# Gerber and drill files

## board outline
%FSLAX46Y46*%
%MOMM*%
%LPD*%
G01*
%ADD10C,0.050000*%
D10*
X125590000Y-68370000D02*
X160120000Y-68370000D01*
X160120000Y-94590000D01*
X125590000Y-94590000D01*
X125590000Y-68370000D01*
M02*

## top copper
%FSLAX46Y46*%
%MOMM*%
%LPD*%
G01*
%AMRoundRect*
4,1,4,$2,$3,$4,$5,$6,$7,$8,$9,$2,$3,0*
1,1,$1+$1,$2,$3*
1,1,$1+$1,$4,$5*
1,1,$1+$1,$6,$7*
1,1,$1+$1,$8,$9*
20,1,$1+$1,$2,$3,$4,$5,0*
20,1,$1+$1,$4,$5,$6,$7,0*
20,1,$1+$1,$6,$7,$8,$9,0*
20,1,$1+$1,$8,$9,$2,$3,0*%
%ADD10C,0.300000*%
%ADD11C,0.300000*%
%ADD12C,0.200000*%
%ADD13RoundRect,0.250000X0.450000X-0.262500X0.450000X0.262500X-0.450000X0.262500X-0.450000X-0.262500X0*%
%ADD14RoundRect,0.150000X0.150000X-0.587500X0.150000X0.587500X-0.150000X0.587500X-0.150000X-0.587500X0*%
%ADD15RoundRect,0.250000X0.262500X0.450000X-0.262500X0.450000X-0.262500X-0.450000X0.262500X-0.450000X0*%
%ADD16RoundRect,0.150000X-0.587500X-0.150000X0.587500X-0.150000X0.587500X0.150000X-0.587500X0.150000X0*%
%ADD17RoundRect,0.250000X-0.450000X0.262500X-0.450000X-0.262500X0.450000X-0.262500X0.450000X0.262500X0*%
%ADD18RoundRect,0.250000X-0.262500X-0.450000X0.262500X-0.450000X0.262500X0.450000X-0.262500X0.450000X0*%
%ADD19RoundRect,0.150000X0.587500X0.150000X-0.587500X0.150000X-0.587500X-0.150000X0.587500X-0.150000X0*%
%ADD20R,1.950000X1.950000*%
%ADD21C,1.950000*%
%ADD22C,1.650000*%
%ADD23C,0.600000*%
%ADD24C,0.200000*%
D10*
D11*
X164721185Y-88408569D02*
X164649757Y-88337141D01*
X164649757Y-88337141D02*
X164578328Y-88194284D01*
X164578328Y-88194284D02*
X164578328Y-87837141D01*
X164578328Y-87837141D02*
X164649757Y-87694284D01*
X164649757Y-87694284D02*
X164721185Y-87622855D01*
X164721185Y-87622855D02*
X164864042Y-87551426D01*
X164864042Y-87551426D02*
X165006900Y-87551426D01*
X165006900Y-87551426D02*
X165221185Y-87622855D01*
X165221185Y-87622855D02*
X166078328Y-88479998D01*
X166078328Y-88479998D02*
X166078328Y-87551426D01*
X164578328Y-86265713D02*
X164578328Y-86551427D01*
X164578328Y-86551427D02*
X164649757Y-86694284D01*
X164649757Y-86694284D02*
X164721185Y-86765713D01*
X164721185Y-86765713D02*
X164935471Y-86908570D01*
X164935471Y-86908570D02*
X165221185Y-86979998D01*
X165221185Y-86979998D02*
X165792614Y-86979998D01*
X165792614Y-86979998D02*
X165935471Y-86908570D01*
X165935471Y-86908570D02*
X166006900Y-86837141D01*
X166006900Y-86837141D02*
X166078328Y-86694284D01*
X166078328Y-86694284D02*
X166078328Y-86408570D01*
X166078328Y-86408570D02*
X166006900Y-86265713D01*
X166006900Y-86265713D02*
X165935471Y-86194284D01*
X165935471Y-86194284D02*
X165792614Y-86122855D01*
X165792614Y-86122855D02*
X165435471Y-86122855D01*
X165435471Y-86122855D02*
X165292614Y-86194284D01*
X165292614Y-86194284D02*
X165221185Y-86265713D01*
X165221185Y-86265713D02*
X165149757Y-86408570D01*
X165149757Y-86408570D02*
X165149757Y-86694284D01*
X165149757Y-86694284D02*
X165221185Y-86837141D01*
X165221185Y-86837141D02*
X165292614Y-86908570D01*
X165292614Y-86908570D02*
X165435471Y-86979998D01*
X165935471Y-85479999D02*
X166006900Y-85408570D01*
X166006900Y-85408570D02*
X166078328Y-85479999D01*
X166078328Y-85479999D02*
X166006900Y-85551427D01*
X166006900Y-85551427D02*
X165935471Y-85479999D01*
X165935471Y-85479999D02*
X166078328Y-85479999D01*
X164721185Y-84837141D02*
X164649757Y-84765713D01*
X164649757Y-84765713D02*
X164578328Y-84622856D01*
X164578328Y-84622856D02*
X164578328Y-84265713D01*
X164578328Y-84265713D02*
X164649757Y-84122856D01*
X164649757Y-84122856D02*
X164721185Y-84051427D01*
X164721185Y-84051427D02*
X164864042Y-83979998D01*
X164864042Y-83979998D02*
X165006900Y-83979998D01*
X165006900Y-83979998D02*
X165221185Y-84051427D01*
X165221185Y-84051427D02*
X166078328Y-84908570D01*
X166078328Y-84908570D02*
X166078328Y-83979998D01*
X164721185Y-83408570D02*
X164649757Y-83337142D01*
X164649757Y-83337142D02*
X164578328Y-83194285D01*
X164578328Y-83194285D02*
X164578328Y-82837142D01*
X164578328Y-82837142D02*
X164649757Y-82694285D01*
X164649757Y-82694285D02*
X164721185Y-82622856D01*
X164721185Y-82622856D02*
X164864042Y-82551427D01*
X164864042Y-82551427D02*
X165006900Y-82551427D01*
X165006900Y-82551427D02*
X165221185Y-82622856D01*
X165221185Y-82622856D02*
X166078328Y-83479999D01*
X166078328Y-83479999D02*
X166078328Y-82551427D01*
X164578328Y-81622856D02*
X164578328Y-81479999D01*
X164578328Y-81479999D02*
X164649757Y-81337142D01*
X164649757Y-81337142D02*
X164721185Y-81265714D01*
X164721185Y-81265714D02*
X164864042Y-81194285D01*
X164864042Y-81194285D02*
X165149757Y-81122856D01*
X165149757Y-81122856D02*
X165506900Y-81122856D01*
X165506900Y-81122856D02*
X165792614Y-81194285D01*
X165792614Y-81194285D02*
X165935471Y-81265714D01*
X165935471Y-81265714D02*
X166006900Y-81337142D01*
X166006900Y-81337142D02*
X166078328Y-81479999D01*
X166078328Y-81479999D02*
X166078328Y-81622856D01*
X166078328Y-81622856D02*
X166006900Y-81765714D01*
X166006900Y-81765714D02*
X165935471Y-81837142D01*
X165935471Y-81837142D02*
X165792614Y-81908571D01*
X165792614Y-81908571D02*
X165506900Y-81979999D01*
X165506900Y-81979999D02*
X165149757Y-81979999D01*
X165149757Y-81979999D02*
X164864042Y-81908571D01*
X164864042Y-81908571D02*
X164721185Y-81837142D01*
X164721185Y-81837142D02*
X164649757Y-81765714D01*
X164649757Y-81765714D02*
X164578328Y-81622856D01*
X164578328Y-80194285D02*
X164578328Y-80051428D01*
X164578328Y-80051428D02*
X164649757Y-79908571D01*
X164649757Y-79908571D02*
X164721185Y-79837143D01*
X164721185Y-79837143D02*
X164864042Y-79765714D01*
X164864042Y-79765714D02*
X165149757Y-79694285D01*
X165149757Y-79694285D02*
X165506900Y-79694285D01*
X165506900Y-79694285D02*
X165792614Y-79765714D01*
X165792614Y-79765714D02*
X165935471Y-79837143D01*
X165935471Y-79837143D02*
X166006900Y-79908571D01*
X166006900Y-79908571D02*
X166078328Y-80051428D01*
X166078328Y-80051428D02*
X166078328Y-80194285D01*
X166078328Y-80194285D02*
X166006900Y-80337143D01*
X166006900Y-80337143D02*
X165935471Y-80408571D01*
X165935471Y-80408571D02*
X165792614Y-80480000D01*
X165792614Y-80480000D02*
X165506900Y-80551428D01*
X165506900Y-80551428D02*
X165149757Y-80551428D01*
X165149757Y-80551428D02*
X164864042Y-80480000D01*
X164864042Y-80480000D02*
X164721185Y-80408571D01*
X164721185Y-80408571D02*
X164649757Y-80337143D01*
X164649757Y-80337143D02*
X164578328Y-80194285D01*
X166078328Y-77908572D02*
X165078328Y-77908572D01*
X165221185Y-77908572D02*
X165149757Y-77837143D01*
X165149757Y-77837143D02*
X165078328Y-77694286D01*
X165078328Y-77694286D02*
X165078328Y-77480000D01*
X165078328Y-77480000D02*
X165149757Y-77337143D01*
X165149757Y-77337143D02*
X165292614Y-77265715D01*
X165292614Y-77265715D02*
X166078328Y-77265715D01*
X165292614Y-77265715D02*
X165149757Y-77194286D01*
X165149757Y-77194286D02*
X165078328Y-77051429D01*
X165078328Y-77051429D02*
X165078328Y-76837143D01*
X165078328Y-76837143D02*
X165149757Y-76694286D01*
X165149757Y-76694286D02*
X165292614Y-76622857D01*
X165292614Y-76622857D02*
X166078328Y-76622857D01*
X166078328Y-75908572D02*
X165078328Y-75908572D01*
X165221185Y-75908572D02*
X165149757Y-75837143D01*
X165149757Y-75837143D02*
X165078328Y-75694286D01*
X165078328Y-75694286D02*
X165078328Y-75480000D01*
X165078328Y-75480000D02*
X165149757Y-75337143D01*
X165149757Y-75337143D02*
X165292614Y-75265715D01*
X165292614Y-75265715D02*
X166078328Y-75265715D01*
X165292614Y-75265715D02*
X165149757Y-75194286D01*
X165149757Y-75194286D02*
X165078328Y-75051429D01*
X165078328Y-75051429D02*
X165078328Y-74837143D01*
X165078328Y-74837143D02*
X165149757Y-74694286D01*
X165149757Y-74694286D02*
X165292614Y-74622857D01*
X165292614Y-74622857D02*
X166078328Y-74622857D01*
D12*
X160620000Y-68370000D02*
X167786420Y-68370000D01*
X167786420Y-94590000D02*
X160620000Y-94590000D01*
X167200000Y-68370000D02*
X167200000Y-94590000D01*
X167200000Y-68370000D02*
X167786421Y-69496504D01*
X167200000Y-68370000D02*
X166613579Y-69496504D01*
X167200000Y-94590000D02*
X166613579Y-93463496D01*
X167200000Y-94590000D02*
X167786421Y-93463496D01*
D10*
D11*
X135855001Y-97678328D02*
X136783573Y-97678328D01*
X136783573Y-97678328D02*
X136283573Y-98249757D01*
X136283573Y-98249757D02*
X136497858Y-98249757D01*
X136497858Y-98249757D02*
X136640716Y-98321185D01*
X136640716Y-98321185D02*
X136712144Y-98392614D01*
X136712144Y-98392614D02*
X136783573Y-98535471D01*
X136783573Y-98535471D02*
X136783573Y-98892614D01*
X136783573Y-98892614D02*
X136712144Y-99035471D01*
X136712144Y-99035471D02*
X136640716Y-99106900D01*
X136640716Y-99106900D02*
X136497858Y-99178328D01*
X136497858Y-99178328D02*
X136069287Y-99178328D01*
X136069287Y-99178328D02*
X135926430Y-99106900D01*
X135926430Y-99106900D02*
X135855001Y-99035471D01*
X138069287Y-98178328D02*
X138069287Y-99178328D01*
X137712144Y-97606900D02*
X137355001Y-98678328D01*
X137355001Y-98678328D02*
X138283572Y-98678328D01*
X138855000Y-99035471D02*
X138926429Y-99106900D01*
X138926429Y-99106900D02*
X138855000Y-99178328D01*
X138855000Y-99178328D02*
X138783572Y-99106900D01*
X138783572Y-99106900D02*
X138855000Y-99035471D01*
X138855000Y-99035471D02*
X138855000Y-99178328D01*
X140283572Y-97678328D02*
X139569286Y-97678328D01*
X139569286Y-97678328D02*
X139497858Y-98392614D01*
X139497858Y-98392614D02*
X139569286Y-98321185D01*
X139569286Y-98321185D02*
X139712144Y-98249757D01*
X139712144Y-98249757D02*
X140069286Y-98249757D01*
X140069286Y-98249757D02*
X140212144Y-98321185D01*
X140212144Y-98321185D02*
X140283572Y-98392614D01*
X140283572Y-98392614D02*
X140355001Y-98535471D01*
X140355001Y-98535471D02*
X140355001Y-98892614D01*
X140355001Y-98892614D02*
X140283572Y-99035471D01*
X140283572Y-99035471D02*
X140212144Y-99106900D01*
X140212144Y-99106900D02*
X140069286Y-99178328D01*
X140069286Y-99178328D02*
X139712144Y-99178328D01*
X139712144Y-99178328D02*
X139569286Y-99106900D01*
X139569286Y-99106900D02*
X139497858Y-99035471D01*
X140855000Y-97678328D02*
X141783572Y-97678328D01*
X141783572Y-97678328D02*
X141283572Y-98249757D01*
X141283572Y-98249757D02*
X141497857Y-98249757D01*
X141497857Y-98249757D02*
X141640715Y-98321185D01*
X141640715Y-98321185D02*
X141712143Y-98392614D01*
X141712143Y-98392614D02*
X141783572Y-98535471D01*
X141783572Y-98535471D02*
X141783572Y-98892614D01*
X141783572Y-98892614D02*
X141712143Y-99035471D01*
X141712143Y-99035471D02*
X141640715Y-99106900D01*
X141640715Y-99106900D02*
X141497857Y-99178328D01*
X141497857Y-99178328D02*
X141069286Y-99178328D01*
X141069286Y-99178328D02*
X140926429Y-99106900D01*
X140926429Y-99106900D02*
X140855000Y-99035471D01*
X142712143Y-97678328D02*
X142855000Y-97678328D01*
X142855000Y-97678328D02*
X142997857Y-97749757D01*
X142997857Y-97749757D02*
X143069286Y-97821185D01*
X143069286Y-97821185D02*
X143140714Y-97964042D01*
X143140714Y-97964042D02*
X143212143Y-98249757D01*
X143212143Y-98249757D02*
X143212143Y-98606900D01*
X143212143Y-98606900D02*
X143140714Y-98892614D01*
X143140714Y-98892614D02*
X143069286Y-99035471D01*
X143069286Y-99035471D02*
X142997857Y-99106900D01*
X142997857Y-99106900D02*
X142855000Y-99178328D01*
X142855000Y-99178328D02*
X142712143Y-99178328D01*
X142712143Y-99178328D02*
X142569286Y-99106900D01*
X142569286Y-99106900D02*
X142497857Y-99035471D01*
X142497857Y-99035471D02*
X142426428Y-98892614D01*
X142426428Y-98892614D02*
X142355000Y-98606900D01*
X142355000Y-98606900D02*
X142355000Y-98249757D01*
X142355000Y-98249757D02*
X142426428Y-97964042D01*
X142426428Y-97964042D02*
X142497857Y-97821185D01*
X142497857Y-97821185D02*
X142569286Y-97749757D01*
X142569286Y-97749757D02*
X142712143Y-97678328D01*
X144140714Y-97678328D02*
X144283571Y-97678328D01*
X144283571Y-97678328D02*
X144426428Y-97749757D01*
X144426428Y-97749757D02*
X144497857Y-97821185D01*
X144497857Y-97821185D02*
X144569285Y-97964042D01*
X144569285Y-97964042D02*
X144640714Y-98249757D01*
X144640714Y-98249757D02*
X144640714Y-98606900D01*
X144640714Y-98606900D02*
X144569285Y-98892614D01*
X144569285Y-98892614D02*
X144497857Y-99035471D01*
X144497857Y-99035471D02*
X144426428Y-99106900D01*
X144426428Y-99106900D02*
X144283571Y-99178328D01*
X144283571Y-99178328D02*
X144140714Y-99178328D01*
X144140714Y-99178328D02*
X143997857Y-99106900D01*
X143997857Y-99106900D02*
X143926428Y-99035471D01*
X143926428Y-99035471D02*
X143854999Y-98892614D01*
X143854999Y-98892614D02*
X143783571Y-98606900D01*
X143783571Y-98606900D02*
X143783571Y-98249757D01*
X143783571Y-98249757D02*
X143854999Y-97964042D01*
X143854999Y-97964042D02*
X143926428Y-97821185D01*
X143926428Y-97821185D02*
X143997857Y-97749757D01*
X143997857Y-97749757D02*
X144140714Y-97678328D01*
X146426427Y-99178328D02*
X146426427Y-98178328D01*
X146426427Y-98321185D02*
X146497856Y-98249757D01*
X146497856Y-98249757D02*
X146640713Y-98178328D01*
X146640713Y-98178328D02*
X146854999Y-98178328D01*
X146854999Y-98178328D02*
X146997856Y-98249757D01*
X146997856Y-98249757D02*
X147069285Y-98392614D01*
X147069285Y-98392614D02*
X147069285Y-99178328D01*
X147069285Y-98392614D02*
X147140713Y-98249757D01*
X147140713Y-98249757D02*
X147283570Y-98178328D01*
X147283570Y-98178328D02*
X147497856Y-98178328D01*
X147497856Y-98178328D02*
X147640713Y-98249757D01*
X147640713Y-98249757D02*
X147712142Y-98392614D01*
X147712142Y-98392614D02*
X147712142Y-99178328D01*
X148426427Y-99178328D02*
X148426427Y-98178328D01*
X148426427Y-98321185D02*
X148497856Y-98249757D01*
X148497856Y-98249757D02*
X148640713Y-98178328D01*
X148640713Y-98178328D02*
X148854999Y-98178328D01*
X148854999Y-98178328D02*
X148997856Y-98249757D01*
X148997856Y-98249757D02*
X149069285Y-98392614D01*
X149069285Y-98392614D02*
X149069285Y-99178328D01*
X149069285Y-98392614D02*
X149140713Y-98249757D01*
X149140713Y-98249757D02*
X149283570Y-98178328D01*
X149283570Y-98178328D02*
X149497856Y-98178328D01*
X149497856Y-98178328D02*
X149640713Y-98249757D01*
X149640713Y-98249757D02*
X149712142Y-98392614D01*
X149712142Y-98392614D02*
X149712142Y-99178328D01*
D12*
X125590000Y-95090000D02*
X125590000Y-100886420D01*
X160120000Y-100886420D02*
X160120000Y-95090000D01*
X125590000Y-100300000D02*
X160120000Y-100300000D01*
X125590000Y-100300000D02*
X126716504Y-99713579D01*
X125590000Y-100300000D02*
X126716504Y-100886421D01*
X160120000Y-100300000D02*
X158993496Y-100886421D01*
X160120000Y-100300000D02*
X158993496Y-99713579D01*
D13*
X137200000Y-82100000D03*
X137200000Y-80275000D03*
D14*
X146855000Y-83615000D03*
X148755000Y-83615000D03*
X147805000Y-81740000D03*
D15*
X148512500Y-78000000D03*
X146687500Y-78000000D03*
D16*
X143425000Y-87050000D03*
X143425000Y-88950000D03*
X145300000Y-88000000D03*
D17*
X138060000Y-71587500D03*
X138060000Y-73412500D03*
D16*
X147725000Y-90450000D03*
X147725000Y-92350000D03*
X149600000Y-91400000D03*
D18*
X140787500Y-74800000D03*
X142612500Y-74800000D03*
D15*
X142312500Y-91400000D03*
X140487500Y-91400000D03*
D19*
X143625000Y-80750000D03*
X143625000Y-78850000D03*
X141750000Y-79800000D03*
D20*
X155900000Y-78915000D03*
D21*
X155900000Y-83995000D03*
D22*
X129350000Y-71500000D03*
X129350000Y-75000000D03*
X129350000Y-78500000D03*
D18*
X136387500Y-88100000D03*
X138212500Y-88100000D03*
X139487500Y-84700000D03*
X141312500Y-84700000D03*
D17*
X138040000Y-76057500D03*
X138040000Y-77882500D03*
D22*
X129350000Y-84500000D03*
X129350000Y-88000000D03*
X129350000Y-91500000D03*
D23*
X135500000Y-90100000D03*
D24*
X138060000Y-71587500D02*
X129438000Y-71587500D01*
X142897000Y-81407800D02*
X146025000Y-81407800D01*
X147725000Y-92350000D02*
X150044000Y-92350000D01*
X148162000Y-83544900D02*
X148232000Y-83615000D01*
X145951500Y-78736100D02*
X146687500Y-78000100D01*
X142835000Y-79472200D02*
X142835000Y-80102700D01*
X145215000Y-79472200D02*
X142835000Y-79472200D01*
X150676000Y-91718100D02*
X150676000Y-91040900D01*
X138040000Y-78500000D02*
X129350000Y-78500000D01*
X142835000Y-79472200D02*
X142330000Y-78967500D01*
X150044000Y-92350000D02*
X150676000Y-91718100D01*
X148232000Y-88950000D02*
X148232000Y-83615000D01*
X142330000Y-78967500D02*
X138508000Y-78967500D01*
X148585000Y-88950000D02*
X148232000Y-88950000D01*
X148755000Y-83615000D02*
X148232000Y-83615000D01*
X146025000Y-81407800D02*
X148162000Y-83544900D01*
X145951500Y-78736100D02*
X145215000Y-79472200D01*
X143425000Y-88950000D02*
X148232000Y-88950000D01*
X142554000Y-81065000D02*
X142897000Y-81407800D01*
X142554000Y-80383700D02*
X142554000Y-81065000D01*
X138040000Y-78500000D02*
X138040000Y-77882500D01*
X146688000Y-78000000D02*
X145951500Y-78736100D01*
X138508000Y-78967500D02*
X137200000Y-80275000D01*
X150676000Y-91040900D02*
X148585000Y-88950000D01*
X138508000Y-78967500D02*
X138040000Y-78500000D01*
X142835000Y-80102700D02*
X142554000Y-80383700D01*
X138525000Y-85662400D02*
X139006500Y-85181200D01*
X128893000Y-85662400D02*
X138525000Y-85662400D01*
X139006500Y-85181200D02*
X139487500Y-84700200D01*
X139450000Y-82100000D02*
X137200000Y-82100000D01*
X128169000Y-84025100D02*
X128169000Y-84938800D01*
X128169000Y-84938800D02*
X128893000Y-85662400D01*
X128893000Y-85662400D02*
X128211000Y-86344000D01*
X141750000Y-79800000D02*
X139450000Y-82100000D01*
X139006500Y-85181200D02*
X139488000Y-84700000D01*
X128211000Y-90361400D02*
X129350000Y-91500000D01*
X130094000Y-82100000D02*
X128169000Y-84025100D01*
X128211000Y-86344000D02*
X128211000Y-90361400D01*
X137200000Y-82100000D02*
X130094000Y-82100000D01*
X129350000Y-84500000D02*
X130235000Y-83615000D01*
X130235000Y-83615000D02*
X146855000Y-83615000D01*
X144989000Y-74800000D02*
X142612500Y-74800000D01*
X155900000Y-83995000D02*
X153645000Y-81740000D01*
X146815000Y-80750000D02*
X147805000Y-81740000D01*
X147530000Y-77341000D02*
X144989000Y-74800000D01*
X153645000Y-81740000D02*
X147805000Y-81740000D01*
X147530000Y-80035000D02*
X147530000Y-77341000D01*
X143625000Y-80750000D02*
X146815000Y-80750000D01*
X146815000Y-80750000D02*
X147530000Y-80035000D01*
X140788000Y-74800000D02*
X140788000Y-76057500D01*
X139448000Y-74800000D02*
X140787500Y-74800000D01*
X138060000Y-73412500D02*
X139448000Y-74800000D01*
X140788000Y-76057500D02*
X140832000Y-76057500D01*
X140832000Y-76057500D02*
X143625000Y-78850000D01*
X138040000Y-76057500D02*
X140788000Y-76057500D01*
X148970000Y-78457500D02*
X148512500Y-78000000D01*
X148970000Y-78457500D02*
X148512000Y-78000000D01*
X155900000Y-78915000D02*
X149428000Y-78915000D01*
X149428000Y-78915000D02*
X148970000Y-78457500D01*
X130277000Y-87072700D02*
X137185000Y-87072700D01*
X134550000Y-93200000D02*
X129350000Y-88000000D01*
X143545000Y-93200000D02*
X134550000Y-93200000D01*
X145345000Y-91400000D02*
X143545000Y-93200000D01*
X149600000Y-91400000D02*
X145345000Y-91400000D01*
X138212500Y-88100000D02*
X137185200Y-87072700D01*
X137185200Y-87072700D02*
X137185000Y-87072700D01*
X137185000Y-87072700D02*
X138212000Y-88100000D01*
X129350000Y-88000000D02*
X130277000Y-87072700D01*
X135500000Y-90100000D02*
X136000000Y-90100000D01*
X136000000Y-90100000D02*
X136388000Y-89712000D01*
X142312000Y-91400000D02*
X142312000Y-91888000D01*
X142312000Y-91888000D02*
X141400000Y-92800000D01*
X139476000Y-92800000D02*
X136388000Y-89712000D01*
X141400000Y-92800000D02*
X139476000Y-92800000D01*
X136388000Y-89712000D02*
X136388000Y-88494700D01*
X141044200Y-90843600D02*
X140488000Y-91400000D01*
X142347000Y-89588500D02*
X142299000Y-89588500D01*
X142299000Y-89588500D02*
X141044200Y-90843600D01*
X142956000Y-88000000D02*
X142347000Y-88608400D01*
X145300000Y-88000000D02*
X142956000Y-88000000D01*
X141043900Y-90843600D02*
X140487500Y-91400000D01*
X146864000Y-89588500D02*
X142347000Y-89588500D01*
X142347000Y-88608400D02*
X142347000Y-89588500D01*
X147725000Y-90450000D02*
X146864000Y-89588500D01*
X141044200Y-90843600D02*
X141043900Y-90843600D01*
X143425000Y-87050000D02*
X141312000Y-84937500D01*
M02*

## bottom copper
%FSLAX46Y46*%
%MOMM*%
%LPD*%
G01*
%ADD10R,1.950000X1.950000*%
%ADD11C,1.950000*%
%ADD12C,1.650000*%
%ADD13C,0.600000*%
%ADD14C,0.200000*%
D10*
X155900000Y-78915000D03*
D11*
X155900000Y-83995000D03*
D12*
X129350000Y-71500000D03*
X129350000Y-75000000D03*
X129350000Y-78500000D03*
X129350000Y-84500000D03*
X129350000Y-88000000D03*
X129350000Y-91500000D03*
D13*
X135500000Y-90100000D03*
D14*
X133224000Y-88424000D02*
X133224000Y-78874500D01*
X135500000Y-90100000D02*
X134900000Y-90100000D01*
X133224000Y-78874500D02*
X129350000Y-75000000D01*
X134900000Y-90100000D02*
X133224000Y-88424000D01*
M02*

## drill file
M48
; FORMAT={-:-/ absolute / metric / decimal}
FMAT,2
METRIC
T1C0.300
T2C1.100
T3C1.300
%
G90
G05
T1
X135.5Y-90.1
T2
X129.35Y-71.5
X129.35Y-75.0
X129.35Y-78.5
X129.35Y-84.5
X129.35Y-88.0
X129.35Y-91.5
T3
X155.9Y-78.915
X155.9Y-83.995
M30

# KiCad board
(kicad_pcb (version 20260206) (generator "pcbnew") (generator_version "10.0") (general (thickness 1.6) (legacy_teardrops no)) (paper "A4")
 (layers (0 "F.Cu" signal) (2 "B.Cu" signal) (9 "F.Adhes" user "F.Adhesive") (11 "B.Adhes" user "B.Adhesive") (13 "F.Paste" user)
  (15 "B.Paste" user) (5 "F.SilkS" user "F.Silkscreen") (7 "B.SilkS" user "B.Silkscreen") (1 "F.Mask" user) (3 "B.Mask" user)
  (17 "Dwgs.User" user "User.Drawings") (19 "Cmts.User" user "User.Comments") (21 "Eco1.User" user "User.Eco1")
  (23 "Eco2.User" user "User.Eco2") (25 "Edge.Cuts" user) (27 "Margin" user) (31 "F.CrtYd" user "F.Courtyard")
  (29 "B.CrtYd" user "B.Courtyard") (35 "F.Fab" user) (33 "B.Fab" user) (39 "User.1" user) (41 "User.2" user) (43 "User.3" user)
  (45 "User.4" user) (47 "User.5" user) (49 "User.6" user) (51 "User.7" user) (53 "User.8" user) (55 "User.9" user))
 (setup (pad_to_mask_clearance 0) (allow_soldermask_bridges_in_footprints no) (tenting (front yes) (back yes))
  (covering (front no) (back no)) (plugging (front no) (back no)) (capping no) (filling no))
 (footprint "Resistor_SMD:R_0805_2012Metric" (layer "F.Cu") (at 137.2 81.1875 90)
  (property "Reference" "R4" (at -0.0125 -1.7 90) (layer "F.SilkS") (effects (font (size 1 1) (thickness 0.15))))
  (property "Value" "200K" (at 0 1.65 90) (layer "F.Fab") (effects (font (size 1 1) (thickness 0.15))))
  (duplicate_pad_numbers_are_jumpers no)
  (pad "1" smd roundrect (at -0.9125 0 90) (size 1.025 1.4) (layers "F.Cu" "F.Mask" "F.Paste") (roundrect_rratio 0.243902) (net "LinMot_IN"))
  (pad "2" smd roundrect (at 0.9125 0 90) (size 1.025 1.4) (layers "F.Cu" "F.Mask" "F.Paste") (roundrect_rratio 0.243902) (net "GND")))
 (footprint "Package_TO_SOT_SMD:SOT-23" (layer "F.Cu") (at 147.805 82.6775 90)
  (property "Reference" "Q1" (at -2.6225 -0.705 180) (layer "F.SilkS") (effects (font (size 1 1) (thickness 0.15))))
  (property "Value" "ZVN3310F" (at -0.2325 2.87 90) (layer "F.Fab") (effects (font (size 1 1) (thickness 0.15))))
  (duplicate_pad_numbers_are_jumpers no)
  (pad "1" smd roundrect (at -0.9375 -0.95 90) (size 1.475 0.6) (layers "F.Cu" "F.Mask" "F.Paste") (roundrect_rratio 0.25)
   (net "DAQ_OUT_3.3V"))
  (pad "2" smd roundrect (at -0.9375 0.95 90) (size 1.475 0.6) (layers "F.Cu" "F.Mask" "F.Paste") (roundrect_rratio 0.25) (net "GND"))
  (pad "3" smd roundrect (at 0.9375 0 90) (size 1.475 0.6) (layers "F.Cu" "F.Mask" "F.Paste") (roundrect_rratio 0.25) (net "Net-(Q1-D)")))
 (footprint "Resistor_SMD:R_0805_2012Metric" (layer "F.Cu") (at 147.6 78 180)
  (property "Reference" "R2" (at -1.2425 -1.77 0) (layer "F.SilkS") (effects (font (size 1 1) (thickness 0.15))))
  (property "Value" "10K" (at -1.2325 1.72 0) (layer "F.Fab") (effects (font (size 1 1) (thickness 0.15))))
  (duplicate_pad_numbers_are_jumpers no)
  (pad "1" smd roundrect (at -0.9125 0 180) (size 1.025 1.4) (layers "F.Cu" "F.Mask" "F.Paste") (roundrect_rratio 0.243902)
   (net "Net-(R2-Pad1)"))
  (pad "2" smd roundrect (at 0.9125 0 180) (size 1.025 1.4) (layers "F.Cu" "F.Mask" "F.Paste") (roundrect_rratio 0.243902) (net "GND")))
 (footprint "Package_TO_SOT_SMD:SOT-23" (layer "F.Cu") (at 144.3625 88)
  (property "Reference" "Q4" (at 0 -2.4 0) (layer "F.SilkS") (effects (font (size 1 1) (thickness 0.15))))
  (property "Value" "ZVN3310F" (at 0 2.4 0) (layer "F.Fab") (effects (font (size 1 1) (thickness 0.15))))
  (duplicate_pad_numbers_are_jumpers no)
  (pad "1" smd roundrect (at -0.9375 -0.95) (size 1.475 0.6) (layers "F.Cu" "F.Mask" "F.Paste") (roundrect_rratio 0.25) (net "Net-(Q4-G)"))
  (pad "2" smd roundrect (at -0.9375 0.95) (size 1.475 0.6) (layers "F.Cu" "F.Mask" "F.Paste") (roundrect_rratio 0.25) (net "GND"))
  (pad "3" smd roundrect (at 0.9375 0) (size 1.475 0.6) (layers "F.Cu" "F.Mask" "F.Paste") (roundrect_rratio 0.25) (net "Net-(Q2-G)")))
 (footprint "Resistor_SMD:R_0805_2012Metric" (layer "F.Cu") (at 138.06 72.5 -90)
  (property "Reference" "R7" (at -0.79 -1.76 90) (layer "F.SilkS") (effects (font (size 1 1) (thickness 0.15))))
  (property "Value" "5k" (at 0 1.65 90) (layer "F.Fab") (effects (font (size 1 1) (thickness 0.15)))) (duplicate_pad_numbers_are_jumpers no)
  (pad "1" smd roundrect (at -0.9125 0 270) (size 1.025 1.4) (layers "F.Cu" "F.Mask" "F.Paste") (roundrect_rratio 0.243902) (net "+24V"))
  (pad "2" smd roundrect (at 0.9125 0 270) (size 1.025 1.4) (layers "F.Cu" "F.Mask" "F.Paste") (roundrect_rratio 0.243902) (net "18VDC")))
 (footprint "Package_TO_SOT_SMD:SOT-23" (layer "F.Cu") (at 148.6625 91.4)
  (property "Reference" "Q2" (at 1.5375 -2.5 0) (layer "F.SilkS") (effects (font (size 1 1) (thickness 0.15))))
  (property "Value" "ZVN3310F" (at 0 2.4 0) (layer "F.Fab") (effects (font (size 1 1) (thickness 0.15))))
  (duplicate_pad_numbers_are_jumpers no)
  (pad "1" smd roundrect (at -0.9375 -0.95) (size 1.475 0.6) (layers "F.Cu" "F.Mask" "F.Paste") (roundrect_rratio 0.25) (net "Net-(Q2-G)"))
  (pad "2" smd roundrect (at -0.9375 0.95) (size 1.475 0.6) (layers "F.Cu" "F.Mask" "F.Paste") (roundrect_rratio 0.25) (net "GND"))
  (pad "3" smd roundrect (at 0.9375 0) (size 1.475 0.6) (layers "F.Cu" "F.Mask" "F.Paste") (roundrect_rratio 0.25) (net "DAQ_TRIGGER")))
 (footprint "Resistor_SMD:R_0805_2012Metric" (layer "F.Cu") (at 141.7 74.8)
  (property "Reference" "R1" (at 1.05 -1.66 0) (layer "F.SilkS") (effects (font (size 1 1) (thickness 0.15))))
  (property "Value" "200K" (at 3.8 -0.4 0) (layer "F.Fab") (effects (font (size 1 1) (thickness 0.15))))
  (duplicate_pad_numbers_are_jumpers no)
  (pad "1" smd roundrect (at -0.9125 0) (size 1.025 1.4) (layers "F.Cu" "F.Mask" "F.Paste") (roundrect_rratio 0.243902) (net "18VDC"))
  (pad "2" smd roundrect (at 0.9125 0) (size 1.025 1.4) (layers "F.Cu" "F.Mask" "F.Paste") (roundrect_rratio 0.243902) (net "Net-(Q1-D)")))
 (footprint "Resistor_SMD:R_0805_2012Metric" (layer "F.Cu") (at 141.4 91.4 180)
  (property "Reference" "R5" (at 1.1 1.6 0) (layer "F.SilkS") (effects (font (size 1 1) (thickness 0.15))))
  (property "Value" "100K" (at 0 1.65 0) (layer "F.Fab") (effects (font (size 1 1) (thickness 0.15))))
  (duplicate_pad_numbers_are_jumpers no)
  (pad "1" smd roundrect (at -0.9125 0 180) (size 1.025 1.4) (layers "F.Cu" "F.Mask" "F.Paste") (roundrect_rratio 0.243902) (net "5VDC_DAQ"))
  (pad "2" smd roundrect (at 0.9125 0 180) (size 1.025 1.4) (layers "F.Cu" "F.Mask" "F.Paste") (roundrect_rratio 0.243902)
   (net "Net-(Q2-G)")))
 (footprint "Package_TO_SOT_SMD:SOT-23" (layer "F.Cu") (at 142.6875 79.8 180)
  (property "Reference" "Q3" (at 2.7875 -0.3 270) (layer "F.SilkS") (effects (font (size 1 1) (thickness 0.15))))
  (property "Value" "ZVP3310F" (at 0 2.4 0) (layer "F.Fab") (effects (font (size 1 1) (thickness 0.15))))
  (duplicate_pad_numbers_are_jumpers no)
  (pad "1" smd roundrect (at -0.9375 -0.95 180) (size 1.475 0.6) (layers "F.Cu" "F.Mask" "F.Paste") (roundrect_rratio 0.25)
   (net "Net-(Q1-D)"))
  (pad "2" smd roundrect (at -0.9375 0.95 180) (size 1.475 0.6) (layers "F.Cu" "F.Mask" "F.Paste") (roundrect_rratio 0.25) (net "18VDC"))
  (pad "3" smd roundrect (at 0.9375 0 180) (size 1.475 0.6) (layers "F.Cu" "F.Mask" "F.Paste") (roundrect_rratio 0.25) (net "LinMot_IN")))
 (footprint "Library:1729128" (layer "F.Cu") (at 155.9 78.915 -90)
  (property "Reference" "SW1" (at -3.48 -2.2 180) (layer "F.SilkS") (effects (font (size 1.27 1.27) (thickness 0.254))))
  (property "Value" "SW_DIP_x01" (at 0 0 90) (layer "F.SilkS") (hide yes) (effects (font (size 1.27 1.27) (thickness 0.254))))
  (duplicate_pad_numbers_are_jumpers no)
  (pad "1" thru_hole rect (at 0 0 270) (size 1.95 1.95) (drill 1.3) (layers "*.Cu" "*.Mask") (remove_unused_layers no) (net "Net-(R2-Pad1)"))
  (pad "2" thru_hole circle (at 5.08 0 270) (size 1.95 1.95) (drill 1.3) (layers "*.Cu" "*.Mask") (remove_unused_layers no)
   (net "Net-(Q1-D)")))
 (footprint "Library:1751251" (layer "F.Cu") (at 129.35 71.5 -90)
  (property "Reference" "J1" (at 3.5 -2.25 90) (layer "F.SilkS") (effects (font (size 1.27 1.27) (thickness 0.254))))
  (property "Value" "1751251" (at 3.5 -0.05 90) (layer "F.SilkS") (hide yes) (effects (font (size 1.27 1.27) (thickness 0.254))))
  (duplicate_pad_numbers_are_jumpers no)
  (pad "1" thru_hole circle (at 0 0 270) (size 1.65 1.65) (drill 1.1) (layers "*.Cu" "*.Mask") (remove_unused_layers no) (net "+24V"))
  (pad "2" thru_hole circle (at 3.5 0 270) (size 1.65 1.65) (drill 1.1) (layers "*.Cu" "*.Mask") (remove_unused_layers no) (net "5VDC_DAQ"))
  (pad "3" thru_hole circle (at 7 0 270) (size 1.65 1.65) (drill 1.1) (layers "*.Cu" "*.Mask") (remove_unused_layers no) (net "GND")))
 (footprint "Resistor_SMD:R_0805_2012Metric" (layer "F.Cu") (at 137.3 88.1)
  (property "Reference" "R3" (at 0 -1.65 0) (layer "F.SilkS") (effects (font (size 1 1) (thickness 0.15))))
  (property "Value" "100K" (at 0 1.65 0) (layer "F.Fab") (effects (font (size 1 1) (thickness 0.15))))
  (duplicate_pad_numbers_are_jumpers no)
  (pad "1" smd roundrect (at -0.9125 0) (size 1.025 1.4) (layers "F.Cu" "F.Mask" "F.Paste") (roundrect_rratio 0.243902) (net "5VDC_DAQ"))
  (pad "2" smd roundrect (at 0.9125 0) (size 1.025 1.4) (layers "F.Cu" "F.Mask" "F.Paste") (roundrect_rratio 0.243902) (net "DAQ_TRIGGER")))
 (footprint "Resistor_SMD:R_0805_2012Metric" (layer "F.Cu") (at 140.4 84.7)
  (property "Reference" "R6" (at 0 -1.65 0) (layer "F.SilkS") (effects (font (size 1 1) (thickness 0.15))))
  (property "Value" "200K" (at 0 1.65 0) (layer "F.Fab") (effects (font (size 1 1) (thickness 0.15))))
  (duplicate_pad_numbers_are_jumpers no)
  (pad "1" smd roundrect (at -0.9125 0) (size 1.025 1.4) (layers "F.Cu" "F.Mask" "F.Paste") (roundrect_rratio 0.243902) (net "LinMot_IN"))
  (pad "2" smd roundrect (at 0.9125 0) (size 1.025 1.4) (layers "F.Cu" "F.Mask" "F.Paste") (roundrect_rratio 0.243902) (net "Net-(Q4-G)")))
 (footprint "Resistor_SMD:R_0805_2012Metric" (layer "F.Cu") (at 138.04 76.97 -90)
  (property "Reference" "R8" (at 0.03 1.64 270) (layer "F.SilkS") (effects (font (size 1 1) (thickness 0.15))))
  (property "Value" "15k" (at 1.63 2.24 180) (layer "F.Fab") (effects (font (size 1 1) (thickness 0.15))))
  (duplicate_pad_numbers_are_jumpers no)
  (pad "1" smd roundrect (at -0.9125 0 270) (size 1.025 1.4) (layers "F.Cu" "F.Mask" "F.Paste") (roundrect_rratio 0.243902) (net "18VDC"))
  (pad "2" smd roundrect (at 0.9125 0 270) (size 1.025 1.4) (layers "F.Cu" "F.Mask" "F.Paste") (roundrect_rratio 0.243902) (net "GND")))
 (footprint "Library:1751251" (layer "F.Cu") (at 129.35 84.5 -90)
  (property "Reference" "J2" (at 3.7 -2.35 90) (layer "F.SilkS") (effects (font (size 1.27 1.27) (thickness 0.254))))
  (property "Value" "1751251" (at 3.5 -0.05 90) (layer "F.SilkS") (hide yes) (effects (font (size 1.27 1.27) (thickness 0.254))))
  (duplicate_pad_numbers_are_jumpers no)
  (pad "1" thru_hole circle (at 0 0 270) (size 1.65 1.65) (drill 1.1) (layers "*.Cu" "*.Mask") (remove_unused_layers no)
   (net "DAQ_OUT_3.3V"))
  (pad "2" thru_hole circle (at 3.5 0 270) (size 1.65 1.65) (drill 1.1) (layers "*.Cu" "*.Mask") (remove_unused_layers no)
   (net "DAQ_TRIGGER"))
  (pad "3" thru_hole circle (at 7 0 270) (size 1.65 1.65) (drill 1.1) (layers "*.Cu" "*.Mask") (remove_unused_layers no) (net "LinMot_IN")))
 (gr_rect (start 125.59 68.37) (end 160.12 94.59) (stroke (width 0.05) (type default)) (fill no) (layer "Edge.Cuts"))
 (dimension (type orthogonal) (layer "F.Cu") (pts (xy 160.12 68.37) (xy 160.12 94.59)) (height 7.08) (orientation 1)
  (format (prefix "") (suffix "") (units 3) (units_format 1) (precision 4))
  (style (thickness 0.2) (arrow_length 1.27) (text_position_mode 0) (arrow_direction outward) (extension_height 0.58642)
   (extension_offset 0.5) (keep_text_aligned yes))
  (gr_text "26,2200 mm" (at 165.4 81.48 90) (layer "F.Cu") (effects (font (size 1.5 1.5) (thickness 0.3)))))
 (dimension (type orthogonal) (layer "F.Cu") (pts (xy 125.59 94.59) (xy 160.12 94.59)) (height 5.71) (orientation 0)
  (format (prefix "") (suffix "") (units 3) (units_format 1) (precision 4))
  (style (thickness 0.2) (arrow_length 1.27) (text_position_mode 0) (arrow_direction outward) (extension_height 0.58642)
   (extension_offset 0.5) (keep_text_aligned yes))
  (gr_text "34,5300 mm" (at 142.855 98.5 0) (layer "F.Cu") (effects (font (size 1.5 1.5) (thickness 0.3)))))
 (segment (start 138.06 71.5875) (end 129.438 71.5875) (width 0.2) (layer "F.Cu") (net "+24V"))
 (segment (start 142.897 81.4078) (end 146.025 81.4078) (width 0.2) (layer "F.Cu") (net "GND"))
 (segment (start 147.725 92.35) (end 150.044 92.35) (width 0.2) (layer "F.Cu") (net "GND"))
 (segment (start 148.162 83.5449) (end 148.232 83.615) (width 0.2) (layer "F.Cu") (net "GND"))
 (segment (start 145.9515 78.7361) (end 146.6875 78.0001) (width 0.2) (layer "F.Cu") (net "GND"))
 (segment (start 142.835 79.4722) (end 142.835 80.1027) (width 0.2) (layer "F.Cu") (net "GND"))
 (segment (start 145.215 79.4722) (end 142.835 79.4722) (width 0.2) (layer "F.Cu") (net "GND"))
 (segment (start 150.676 91.7181) (end 150.676 91.0409) (width 0.2) (layer "F.Cu") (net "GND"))
 (segment (start 138.04 78.5) (end 129.35 78.5) (width 0.2) (layer "F.Cu") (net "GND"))
 (segment (start 142.835 79.4722) (end 142.33 78.9675) (width 0.2) (layer "F.Cu") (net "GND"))
 (segment (start 150.044 92.35) (end 150.676 91.7181) (width 0.2) (layer "F.Cu") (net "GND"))
 (segment (start 148.232 88.95) (end 148.232 83.615) (width 0.2) (layer "F.Cu") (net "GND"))
 (segment (start 142.33 78.9675) (end 138.508 78.9675) (width 0.2) (layer "F.Cu") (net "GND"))
 (segment (start 148.585 88.95) (end 148.232 88.95) (width 0.2) (layer "F.Cu") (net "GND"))
 (segment (start 148.755 83.615) (end 148.232 83.615) (width 0.2) (layer "F.Cu") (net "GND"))
 (segment (start 146.025 81.4078) (end 148.162 83.5449) (width 0.2) (layer "F.Cu") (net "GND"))
 (segment (start 145.9515 78.7361) (end 145.215 79.4722) (width 0.2) (layer "F.Cu") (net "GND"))
 (segment (start 143.425 88.95) (end 148.232 88.95) (width 0.2) (layer "F.Cu") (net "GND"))
 (segment (start 142.554 81.065) (end 142.897 81.4078) (width 0.2) (layer "F.Cu") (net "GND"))
 (segment (start 142.554 80.3837) (end 142.554 81.065) (width 0.2) (layer "F.Cu") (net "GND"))
 (segment (start 138.04 78.5) (end 138.04 77.8825) (width 0.2) (layer "F.Cu") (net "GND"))
 (segment (start 146.688 78) (end 145.9515 78.7361) (width 0.2) (layer "F.Cu") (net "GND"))
 (segment (start 138.508 78.9675) (end 137.2 80.275) (width 0.2) (layer "F.Cu") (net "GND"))
 (segment (start 150.676 91.0409) (end 148.585 88.95) (width 0.2) (layer "F.Cu") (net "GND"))
 (segment (start 138.508 78.9675) (end 138.04 78.5) (width 0.2) (layer "F.Cu") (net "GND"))
 (segment (start 142.835 80.1027) (end 142.554 80.3837) (width 0.2) (layer "F.Cu") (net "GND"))
 (segment (start 138.525 85.6624) (end 139.0065 85.1812) (width 0.2) (layer "F.Cu") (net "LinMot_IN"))
 (segment (start 128.893 85.6624) (end 138.525 85.6624) (width 0.2) (layer "F.Cu") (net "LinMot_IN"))
 (segment (start 139.0065 85.1812) (end 139.4875 84.7002) (width 0.2) (layer "F.Cu") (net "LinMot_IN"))
 (segment (start 139.45 82.1) (end 137.2 82.1) (width 0.2) (layer "F.Cu") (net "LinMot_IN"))
 (segment (start 128.169 84.0251) (end 128.169 84.9388) (width 0.2) (layer "F.Cu") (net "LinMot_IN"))
 (segment (start 128.169 84.9388) (end 128.893 85.6624) (width 0.2) (layer "F.Cu") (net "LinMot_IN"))
 (segment (start 128.893 85.6624) (end 128.211 86.344) (width 0.2) (layer "F.Cu") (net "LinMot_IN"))
 (segment (start 141.75 79.8) (end 139.45 82.1) (width 0.2) (layer "F.Cu") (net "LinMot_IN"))
 (segment (start 139.0065 85.1812) (end 139.488 84.7) (width 0.2) (layer "F.Cu") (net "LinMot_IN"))
 (segment (start 128.211 90.3614) (end 129.35 91.5) (width 0.2) (layer "F.Cu") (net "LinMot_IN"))
 (segment (start 130.094 82.1) (end 128.169 84.0251) (width 0.2) (layer "F.Cu") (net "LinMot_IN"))
 (segment (start 128.211 86.344) (end 128.211 90.3614) (width 0.2) (layer "F.Cu") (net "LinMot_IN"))
 (segment (start 137.2 82.1) (end 130.094 82.1) (width 0.2) (layer "F.Cu") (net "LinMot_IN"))
 (segment (start 129.35 84.5) (end 130.235 83.615) (width 0.2) (layer "F.Cu") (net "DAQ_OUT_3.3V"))
 (segment (start 130.235 83.615) (end 146.855 83.615) (width 0.2) (layer "F.Cu") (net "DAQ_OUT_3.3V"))
 (segment (start 144.989 74.8) (end 142.6125 74.8) (width 0.2) (layer "F.Cu") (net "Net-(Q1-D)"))
 (segment (start 155.9 83.995) (end 153.645 81.74) (width 0.2) (layer "F.Cu") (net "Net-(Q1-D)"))
 (segment (start 146.815 80.75) (end 147.805 81.74) (width 0.2) (layer "F.Cu") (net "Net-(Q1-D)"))
 (segment (start 147.53 77.341) (end 144.989 74.8) (width 0.2) (layer "F.Cu") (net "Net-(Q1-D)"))
 (segment (start 153.645 81.74) (end 147.805 81.74) (width 0.2) (layer "F.Cu") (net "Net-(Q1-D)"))
 (segment (start 147.53 80.035) (end 147.53 77.341) (width 0.2) (layer "F.Cu") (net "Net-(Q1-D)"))
 (segment (start 143.625 80.75) (end 146.815 80.75) (width 0.2) (layer "F.Cu") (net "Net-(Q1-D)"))
 (segment (start 146.815 80.75) (end 147.53 80.035) (width 0.2) (layer "F.Cu") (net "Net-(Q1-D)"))
 (segment (start 140.788 74.8) (end 140.788 76.0575) (width 0.2) (layer "F.Cu") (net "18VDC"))
 (segment (start 139.448 74.8) (end 140.7875 74.8) (width 0.2) (layer "F.Cu") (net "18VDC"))
 (segment (start 138.06 73.4125) (end 139.448 74.8) (width 0.2) (layer "F.Cu") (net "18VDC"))
 (segment (start 140.788 76.0575) (end 140.832 76.0575) (width 0.2) (layer "F.Cu") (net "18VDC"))
 (segment (start 140.832 76.0575) (end 143.625 78.85) (width 0.2) (layer "F.Cu") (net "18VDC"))
 (segment (start 138.04 76.0575) (end 140.788 76.0575) (width 0.2) (layer "F.Cu") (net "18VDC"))
 (segment (start 148.97 78.4575) (end 148.5125 78) (width 0.2) (layer "F.Cu") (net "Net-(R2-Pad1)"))
 (segment (start 148.97 78.4575) (end 148.512 78) (width 0.2) (layer "F.Cu") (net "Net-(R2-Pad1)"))
 (segment (start 155.9 78.915) (end 149.428 78.915) (width 0.2) (layer "F.Cu") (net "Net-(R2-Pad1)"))
 (segment (start 149.428 78.915) (end 148.97 78.4575) (width 0.2) (layer "F.Cu") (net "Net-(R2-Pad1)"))
 (segment (start 130.277 87.0727) (end 137.185 87.0727) (width 0.2) (layer "F.Cu") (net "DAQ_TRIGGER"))
 (segment (start 134.55 93.2) (end 129.35 88) (width 0.2) (layer "F.Cu") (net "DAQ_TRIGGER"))
 (segment (start 143.545 93.2) (end 134.55 93.2) (width 0.2) (layer "F.Cu") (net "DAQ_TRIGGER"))
 (segment (start 145.345 91.4) (end 143.545 93.2) (width 0.2) (layer "F.Cu") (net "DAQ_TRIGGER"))
 (segment (start 149.6 91.4) (end 145.345 91.4) (width 0.2) (layer "F.Cu") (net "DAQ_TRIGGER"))
 (segment (start 138.2125 88.1) (end 137.1852 87.0727) (width 0.2) (layer "F.Cu") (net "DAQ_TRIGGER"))
 (segment (start 137.1852 87.0727) (end 137.185 87.0727) (width 0.2) (layer "F.Cu") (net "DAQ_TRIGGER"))
 (segment (start 137.185 87.0727) (end 138.212 88.1) (width 0.2) (layer "F.Cu") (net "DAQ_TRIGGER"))
 (segment (start 129.35 88) (end 130.277 87.0727) (width 0.2) (layer "F.Cu") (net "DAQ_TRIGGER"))
 (segment (start 135.5 90.1) (end 136 90.1) (width 0.2) (layer "F.Cu") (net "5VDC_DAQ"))
 (segment (start 136 90.1) (end 136.388 89.712) (width 0.2) (layer "F.Cu") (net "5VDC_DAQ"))
 (segment (start 142.312 91.4) (end 142.312 91.888) (width 0.2) (layer "F.Cu") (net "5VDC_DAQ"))
 (segment (start 142.312 91.888) (end 141.4 92.8) (width 0.2) (layer "F.Cu") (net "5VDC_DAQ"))
 (segment (start 139.476 92.8) (end 136.388 89.712) (width 0.2) (layer "F.Cu") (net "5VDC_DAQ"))
 (segment (start 141.4 92.8) (end 139.476 92.8) (width 0.2) (layer "F.Cu") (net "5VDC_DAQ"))
 (segment (start 136.388 89.712) (end 136.388 88.4947) (width 0.2) (layer "F.Cu") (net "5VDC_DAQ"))
 (via (at 135.5 90.1) (size 0.6) (drill 0.3) (layers "F.Cu" "B.Cu") (capping no) (covering (front no) (back no))
  (plugging (front no) (back no)) (filling no) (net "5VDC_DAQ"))
 (segment (start 133.224 88.424) (end 133.224 78.8745) (width 0.2) (layer "B.Cu") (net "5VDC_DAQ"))
 (segment (start 135.5 90.1) (end 134.9 90.1) (width 0.2) (layer "B.Cu") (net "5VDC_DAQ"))
 (segment (start 133.224 78.8745) (end 129.35 75) (width 0.2) (layer "B.Cu") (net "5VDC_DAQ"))
 (segment (start 134.9 90.1) (end 133.224 88.424) (width 0.2) (layer "B.Cu") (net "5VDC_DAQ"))
 (segment (start 141.0442 90.8436) (end 140.488 91.4) (width 0.2) (layer "F.Cu") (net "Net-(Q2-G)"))
 (segment (start 142.347 89.5885) (end 142.299 89.5885) (width 0.2) (layer "F.Cu") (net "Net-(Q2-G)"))
 (segment (start 142.299 89.5885) (end 141.0442 90.8436) (width 0.2) (layer "F.Cu") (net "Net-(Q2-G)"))
 (segment (start 142.956 88) (end 142.347 88.6084) (width 0.2) (layer "F.Cu") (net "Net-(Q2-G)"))
 (segment (start 145.3 88) (end 142.956 88) (width 0.2) (layer "F.Cu") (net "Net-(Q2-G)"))
 (segment (start 141.0439 90.8436) (end 140.4875 91.4) (width 0.2) (layer "F.Cu") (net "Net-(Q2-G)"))
 (segment (start 146.864 89.5885) (end 142.347 89.5885) (width 0.2) (layer "F.Cu") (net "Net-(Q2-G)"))
 (segment (start 142.347 88.6084) (end 142.347 89.5885) (width 0.2) (layer "F.Cu") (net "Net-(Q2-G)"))
 (segment (start 147.725 90.45) (end 146.864 89.5885) (width 0.2) (layer "F.Cu") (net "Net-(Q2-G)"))
 (segment (start 141.0442 90.8436) (end 141.0439 90.8436) (width 0.2) (layer "F.Cu") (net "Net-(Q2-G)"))
 (segment (start 143.425 87.05) (end 141.312 84.9375) (width 0.2) (layer "F.Cu") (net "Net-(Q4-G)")))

